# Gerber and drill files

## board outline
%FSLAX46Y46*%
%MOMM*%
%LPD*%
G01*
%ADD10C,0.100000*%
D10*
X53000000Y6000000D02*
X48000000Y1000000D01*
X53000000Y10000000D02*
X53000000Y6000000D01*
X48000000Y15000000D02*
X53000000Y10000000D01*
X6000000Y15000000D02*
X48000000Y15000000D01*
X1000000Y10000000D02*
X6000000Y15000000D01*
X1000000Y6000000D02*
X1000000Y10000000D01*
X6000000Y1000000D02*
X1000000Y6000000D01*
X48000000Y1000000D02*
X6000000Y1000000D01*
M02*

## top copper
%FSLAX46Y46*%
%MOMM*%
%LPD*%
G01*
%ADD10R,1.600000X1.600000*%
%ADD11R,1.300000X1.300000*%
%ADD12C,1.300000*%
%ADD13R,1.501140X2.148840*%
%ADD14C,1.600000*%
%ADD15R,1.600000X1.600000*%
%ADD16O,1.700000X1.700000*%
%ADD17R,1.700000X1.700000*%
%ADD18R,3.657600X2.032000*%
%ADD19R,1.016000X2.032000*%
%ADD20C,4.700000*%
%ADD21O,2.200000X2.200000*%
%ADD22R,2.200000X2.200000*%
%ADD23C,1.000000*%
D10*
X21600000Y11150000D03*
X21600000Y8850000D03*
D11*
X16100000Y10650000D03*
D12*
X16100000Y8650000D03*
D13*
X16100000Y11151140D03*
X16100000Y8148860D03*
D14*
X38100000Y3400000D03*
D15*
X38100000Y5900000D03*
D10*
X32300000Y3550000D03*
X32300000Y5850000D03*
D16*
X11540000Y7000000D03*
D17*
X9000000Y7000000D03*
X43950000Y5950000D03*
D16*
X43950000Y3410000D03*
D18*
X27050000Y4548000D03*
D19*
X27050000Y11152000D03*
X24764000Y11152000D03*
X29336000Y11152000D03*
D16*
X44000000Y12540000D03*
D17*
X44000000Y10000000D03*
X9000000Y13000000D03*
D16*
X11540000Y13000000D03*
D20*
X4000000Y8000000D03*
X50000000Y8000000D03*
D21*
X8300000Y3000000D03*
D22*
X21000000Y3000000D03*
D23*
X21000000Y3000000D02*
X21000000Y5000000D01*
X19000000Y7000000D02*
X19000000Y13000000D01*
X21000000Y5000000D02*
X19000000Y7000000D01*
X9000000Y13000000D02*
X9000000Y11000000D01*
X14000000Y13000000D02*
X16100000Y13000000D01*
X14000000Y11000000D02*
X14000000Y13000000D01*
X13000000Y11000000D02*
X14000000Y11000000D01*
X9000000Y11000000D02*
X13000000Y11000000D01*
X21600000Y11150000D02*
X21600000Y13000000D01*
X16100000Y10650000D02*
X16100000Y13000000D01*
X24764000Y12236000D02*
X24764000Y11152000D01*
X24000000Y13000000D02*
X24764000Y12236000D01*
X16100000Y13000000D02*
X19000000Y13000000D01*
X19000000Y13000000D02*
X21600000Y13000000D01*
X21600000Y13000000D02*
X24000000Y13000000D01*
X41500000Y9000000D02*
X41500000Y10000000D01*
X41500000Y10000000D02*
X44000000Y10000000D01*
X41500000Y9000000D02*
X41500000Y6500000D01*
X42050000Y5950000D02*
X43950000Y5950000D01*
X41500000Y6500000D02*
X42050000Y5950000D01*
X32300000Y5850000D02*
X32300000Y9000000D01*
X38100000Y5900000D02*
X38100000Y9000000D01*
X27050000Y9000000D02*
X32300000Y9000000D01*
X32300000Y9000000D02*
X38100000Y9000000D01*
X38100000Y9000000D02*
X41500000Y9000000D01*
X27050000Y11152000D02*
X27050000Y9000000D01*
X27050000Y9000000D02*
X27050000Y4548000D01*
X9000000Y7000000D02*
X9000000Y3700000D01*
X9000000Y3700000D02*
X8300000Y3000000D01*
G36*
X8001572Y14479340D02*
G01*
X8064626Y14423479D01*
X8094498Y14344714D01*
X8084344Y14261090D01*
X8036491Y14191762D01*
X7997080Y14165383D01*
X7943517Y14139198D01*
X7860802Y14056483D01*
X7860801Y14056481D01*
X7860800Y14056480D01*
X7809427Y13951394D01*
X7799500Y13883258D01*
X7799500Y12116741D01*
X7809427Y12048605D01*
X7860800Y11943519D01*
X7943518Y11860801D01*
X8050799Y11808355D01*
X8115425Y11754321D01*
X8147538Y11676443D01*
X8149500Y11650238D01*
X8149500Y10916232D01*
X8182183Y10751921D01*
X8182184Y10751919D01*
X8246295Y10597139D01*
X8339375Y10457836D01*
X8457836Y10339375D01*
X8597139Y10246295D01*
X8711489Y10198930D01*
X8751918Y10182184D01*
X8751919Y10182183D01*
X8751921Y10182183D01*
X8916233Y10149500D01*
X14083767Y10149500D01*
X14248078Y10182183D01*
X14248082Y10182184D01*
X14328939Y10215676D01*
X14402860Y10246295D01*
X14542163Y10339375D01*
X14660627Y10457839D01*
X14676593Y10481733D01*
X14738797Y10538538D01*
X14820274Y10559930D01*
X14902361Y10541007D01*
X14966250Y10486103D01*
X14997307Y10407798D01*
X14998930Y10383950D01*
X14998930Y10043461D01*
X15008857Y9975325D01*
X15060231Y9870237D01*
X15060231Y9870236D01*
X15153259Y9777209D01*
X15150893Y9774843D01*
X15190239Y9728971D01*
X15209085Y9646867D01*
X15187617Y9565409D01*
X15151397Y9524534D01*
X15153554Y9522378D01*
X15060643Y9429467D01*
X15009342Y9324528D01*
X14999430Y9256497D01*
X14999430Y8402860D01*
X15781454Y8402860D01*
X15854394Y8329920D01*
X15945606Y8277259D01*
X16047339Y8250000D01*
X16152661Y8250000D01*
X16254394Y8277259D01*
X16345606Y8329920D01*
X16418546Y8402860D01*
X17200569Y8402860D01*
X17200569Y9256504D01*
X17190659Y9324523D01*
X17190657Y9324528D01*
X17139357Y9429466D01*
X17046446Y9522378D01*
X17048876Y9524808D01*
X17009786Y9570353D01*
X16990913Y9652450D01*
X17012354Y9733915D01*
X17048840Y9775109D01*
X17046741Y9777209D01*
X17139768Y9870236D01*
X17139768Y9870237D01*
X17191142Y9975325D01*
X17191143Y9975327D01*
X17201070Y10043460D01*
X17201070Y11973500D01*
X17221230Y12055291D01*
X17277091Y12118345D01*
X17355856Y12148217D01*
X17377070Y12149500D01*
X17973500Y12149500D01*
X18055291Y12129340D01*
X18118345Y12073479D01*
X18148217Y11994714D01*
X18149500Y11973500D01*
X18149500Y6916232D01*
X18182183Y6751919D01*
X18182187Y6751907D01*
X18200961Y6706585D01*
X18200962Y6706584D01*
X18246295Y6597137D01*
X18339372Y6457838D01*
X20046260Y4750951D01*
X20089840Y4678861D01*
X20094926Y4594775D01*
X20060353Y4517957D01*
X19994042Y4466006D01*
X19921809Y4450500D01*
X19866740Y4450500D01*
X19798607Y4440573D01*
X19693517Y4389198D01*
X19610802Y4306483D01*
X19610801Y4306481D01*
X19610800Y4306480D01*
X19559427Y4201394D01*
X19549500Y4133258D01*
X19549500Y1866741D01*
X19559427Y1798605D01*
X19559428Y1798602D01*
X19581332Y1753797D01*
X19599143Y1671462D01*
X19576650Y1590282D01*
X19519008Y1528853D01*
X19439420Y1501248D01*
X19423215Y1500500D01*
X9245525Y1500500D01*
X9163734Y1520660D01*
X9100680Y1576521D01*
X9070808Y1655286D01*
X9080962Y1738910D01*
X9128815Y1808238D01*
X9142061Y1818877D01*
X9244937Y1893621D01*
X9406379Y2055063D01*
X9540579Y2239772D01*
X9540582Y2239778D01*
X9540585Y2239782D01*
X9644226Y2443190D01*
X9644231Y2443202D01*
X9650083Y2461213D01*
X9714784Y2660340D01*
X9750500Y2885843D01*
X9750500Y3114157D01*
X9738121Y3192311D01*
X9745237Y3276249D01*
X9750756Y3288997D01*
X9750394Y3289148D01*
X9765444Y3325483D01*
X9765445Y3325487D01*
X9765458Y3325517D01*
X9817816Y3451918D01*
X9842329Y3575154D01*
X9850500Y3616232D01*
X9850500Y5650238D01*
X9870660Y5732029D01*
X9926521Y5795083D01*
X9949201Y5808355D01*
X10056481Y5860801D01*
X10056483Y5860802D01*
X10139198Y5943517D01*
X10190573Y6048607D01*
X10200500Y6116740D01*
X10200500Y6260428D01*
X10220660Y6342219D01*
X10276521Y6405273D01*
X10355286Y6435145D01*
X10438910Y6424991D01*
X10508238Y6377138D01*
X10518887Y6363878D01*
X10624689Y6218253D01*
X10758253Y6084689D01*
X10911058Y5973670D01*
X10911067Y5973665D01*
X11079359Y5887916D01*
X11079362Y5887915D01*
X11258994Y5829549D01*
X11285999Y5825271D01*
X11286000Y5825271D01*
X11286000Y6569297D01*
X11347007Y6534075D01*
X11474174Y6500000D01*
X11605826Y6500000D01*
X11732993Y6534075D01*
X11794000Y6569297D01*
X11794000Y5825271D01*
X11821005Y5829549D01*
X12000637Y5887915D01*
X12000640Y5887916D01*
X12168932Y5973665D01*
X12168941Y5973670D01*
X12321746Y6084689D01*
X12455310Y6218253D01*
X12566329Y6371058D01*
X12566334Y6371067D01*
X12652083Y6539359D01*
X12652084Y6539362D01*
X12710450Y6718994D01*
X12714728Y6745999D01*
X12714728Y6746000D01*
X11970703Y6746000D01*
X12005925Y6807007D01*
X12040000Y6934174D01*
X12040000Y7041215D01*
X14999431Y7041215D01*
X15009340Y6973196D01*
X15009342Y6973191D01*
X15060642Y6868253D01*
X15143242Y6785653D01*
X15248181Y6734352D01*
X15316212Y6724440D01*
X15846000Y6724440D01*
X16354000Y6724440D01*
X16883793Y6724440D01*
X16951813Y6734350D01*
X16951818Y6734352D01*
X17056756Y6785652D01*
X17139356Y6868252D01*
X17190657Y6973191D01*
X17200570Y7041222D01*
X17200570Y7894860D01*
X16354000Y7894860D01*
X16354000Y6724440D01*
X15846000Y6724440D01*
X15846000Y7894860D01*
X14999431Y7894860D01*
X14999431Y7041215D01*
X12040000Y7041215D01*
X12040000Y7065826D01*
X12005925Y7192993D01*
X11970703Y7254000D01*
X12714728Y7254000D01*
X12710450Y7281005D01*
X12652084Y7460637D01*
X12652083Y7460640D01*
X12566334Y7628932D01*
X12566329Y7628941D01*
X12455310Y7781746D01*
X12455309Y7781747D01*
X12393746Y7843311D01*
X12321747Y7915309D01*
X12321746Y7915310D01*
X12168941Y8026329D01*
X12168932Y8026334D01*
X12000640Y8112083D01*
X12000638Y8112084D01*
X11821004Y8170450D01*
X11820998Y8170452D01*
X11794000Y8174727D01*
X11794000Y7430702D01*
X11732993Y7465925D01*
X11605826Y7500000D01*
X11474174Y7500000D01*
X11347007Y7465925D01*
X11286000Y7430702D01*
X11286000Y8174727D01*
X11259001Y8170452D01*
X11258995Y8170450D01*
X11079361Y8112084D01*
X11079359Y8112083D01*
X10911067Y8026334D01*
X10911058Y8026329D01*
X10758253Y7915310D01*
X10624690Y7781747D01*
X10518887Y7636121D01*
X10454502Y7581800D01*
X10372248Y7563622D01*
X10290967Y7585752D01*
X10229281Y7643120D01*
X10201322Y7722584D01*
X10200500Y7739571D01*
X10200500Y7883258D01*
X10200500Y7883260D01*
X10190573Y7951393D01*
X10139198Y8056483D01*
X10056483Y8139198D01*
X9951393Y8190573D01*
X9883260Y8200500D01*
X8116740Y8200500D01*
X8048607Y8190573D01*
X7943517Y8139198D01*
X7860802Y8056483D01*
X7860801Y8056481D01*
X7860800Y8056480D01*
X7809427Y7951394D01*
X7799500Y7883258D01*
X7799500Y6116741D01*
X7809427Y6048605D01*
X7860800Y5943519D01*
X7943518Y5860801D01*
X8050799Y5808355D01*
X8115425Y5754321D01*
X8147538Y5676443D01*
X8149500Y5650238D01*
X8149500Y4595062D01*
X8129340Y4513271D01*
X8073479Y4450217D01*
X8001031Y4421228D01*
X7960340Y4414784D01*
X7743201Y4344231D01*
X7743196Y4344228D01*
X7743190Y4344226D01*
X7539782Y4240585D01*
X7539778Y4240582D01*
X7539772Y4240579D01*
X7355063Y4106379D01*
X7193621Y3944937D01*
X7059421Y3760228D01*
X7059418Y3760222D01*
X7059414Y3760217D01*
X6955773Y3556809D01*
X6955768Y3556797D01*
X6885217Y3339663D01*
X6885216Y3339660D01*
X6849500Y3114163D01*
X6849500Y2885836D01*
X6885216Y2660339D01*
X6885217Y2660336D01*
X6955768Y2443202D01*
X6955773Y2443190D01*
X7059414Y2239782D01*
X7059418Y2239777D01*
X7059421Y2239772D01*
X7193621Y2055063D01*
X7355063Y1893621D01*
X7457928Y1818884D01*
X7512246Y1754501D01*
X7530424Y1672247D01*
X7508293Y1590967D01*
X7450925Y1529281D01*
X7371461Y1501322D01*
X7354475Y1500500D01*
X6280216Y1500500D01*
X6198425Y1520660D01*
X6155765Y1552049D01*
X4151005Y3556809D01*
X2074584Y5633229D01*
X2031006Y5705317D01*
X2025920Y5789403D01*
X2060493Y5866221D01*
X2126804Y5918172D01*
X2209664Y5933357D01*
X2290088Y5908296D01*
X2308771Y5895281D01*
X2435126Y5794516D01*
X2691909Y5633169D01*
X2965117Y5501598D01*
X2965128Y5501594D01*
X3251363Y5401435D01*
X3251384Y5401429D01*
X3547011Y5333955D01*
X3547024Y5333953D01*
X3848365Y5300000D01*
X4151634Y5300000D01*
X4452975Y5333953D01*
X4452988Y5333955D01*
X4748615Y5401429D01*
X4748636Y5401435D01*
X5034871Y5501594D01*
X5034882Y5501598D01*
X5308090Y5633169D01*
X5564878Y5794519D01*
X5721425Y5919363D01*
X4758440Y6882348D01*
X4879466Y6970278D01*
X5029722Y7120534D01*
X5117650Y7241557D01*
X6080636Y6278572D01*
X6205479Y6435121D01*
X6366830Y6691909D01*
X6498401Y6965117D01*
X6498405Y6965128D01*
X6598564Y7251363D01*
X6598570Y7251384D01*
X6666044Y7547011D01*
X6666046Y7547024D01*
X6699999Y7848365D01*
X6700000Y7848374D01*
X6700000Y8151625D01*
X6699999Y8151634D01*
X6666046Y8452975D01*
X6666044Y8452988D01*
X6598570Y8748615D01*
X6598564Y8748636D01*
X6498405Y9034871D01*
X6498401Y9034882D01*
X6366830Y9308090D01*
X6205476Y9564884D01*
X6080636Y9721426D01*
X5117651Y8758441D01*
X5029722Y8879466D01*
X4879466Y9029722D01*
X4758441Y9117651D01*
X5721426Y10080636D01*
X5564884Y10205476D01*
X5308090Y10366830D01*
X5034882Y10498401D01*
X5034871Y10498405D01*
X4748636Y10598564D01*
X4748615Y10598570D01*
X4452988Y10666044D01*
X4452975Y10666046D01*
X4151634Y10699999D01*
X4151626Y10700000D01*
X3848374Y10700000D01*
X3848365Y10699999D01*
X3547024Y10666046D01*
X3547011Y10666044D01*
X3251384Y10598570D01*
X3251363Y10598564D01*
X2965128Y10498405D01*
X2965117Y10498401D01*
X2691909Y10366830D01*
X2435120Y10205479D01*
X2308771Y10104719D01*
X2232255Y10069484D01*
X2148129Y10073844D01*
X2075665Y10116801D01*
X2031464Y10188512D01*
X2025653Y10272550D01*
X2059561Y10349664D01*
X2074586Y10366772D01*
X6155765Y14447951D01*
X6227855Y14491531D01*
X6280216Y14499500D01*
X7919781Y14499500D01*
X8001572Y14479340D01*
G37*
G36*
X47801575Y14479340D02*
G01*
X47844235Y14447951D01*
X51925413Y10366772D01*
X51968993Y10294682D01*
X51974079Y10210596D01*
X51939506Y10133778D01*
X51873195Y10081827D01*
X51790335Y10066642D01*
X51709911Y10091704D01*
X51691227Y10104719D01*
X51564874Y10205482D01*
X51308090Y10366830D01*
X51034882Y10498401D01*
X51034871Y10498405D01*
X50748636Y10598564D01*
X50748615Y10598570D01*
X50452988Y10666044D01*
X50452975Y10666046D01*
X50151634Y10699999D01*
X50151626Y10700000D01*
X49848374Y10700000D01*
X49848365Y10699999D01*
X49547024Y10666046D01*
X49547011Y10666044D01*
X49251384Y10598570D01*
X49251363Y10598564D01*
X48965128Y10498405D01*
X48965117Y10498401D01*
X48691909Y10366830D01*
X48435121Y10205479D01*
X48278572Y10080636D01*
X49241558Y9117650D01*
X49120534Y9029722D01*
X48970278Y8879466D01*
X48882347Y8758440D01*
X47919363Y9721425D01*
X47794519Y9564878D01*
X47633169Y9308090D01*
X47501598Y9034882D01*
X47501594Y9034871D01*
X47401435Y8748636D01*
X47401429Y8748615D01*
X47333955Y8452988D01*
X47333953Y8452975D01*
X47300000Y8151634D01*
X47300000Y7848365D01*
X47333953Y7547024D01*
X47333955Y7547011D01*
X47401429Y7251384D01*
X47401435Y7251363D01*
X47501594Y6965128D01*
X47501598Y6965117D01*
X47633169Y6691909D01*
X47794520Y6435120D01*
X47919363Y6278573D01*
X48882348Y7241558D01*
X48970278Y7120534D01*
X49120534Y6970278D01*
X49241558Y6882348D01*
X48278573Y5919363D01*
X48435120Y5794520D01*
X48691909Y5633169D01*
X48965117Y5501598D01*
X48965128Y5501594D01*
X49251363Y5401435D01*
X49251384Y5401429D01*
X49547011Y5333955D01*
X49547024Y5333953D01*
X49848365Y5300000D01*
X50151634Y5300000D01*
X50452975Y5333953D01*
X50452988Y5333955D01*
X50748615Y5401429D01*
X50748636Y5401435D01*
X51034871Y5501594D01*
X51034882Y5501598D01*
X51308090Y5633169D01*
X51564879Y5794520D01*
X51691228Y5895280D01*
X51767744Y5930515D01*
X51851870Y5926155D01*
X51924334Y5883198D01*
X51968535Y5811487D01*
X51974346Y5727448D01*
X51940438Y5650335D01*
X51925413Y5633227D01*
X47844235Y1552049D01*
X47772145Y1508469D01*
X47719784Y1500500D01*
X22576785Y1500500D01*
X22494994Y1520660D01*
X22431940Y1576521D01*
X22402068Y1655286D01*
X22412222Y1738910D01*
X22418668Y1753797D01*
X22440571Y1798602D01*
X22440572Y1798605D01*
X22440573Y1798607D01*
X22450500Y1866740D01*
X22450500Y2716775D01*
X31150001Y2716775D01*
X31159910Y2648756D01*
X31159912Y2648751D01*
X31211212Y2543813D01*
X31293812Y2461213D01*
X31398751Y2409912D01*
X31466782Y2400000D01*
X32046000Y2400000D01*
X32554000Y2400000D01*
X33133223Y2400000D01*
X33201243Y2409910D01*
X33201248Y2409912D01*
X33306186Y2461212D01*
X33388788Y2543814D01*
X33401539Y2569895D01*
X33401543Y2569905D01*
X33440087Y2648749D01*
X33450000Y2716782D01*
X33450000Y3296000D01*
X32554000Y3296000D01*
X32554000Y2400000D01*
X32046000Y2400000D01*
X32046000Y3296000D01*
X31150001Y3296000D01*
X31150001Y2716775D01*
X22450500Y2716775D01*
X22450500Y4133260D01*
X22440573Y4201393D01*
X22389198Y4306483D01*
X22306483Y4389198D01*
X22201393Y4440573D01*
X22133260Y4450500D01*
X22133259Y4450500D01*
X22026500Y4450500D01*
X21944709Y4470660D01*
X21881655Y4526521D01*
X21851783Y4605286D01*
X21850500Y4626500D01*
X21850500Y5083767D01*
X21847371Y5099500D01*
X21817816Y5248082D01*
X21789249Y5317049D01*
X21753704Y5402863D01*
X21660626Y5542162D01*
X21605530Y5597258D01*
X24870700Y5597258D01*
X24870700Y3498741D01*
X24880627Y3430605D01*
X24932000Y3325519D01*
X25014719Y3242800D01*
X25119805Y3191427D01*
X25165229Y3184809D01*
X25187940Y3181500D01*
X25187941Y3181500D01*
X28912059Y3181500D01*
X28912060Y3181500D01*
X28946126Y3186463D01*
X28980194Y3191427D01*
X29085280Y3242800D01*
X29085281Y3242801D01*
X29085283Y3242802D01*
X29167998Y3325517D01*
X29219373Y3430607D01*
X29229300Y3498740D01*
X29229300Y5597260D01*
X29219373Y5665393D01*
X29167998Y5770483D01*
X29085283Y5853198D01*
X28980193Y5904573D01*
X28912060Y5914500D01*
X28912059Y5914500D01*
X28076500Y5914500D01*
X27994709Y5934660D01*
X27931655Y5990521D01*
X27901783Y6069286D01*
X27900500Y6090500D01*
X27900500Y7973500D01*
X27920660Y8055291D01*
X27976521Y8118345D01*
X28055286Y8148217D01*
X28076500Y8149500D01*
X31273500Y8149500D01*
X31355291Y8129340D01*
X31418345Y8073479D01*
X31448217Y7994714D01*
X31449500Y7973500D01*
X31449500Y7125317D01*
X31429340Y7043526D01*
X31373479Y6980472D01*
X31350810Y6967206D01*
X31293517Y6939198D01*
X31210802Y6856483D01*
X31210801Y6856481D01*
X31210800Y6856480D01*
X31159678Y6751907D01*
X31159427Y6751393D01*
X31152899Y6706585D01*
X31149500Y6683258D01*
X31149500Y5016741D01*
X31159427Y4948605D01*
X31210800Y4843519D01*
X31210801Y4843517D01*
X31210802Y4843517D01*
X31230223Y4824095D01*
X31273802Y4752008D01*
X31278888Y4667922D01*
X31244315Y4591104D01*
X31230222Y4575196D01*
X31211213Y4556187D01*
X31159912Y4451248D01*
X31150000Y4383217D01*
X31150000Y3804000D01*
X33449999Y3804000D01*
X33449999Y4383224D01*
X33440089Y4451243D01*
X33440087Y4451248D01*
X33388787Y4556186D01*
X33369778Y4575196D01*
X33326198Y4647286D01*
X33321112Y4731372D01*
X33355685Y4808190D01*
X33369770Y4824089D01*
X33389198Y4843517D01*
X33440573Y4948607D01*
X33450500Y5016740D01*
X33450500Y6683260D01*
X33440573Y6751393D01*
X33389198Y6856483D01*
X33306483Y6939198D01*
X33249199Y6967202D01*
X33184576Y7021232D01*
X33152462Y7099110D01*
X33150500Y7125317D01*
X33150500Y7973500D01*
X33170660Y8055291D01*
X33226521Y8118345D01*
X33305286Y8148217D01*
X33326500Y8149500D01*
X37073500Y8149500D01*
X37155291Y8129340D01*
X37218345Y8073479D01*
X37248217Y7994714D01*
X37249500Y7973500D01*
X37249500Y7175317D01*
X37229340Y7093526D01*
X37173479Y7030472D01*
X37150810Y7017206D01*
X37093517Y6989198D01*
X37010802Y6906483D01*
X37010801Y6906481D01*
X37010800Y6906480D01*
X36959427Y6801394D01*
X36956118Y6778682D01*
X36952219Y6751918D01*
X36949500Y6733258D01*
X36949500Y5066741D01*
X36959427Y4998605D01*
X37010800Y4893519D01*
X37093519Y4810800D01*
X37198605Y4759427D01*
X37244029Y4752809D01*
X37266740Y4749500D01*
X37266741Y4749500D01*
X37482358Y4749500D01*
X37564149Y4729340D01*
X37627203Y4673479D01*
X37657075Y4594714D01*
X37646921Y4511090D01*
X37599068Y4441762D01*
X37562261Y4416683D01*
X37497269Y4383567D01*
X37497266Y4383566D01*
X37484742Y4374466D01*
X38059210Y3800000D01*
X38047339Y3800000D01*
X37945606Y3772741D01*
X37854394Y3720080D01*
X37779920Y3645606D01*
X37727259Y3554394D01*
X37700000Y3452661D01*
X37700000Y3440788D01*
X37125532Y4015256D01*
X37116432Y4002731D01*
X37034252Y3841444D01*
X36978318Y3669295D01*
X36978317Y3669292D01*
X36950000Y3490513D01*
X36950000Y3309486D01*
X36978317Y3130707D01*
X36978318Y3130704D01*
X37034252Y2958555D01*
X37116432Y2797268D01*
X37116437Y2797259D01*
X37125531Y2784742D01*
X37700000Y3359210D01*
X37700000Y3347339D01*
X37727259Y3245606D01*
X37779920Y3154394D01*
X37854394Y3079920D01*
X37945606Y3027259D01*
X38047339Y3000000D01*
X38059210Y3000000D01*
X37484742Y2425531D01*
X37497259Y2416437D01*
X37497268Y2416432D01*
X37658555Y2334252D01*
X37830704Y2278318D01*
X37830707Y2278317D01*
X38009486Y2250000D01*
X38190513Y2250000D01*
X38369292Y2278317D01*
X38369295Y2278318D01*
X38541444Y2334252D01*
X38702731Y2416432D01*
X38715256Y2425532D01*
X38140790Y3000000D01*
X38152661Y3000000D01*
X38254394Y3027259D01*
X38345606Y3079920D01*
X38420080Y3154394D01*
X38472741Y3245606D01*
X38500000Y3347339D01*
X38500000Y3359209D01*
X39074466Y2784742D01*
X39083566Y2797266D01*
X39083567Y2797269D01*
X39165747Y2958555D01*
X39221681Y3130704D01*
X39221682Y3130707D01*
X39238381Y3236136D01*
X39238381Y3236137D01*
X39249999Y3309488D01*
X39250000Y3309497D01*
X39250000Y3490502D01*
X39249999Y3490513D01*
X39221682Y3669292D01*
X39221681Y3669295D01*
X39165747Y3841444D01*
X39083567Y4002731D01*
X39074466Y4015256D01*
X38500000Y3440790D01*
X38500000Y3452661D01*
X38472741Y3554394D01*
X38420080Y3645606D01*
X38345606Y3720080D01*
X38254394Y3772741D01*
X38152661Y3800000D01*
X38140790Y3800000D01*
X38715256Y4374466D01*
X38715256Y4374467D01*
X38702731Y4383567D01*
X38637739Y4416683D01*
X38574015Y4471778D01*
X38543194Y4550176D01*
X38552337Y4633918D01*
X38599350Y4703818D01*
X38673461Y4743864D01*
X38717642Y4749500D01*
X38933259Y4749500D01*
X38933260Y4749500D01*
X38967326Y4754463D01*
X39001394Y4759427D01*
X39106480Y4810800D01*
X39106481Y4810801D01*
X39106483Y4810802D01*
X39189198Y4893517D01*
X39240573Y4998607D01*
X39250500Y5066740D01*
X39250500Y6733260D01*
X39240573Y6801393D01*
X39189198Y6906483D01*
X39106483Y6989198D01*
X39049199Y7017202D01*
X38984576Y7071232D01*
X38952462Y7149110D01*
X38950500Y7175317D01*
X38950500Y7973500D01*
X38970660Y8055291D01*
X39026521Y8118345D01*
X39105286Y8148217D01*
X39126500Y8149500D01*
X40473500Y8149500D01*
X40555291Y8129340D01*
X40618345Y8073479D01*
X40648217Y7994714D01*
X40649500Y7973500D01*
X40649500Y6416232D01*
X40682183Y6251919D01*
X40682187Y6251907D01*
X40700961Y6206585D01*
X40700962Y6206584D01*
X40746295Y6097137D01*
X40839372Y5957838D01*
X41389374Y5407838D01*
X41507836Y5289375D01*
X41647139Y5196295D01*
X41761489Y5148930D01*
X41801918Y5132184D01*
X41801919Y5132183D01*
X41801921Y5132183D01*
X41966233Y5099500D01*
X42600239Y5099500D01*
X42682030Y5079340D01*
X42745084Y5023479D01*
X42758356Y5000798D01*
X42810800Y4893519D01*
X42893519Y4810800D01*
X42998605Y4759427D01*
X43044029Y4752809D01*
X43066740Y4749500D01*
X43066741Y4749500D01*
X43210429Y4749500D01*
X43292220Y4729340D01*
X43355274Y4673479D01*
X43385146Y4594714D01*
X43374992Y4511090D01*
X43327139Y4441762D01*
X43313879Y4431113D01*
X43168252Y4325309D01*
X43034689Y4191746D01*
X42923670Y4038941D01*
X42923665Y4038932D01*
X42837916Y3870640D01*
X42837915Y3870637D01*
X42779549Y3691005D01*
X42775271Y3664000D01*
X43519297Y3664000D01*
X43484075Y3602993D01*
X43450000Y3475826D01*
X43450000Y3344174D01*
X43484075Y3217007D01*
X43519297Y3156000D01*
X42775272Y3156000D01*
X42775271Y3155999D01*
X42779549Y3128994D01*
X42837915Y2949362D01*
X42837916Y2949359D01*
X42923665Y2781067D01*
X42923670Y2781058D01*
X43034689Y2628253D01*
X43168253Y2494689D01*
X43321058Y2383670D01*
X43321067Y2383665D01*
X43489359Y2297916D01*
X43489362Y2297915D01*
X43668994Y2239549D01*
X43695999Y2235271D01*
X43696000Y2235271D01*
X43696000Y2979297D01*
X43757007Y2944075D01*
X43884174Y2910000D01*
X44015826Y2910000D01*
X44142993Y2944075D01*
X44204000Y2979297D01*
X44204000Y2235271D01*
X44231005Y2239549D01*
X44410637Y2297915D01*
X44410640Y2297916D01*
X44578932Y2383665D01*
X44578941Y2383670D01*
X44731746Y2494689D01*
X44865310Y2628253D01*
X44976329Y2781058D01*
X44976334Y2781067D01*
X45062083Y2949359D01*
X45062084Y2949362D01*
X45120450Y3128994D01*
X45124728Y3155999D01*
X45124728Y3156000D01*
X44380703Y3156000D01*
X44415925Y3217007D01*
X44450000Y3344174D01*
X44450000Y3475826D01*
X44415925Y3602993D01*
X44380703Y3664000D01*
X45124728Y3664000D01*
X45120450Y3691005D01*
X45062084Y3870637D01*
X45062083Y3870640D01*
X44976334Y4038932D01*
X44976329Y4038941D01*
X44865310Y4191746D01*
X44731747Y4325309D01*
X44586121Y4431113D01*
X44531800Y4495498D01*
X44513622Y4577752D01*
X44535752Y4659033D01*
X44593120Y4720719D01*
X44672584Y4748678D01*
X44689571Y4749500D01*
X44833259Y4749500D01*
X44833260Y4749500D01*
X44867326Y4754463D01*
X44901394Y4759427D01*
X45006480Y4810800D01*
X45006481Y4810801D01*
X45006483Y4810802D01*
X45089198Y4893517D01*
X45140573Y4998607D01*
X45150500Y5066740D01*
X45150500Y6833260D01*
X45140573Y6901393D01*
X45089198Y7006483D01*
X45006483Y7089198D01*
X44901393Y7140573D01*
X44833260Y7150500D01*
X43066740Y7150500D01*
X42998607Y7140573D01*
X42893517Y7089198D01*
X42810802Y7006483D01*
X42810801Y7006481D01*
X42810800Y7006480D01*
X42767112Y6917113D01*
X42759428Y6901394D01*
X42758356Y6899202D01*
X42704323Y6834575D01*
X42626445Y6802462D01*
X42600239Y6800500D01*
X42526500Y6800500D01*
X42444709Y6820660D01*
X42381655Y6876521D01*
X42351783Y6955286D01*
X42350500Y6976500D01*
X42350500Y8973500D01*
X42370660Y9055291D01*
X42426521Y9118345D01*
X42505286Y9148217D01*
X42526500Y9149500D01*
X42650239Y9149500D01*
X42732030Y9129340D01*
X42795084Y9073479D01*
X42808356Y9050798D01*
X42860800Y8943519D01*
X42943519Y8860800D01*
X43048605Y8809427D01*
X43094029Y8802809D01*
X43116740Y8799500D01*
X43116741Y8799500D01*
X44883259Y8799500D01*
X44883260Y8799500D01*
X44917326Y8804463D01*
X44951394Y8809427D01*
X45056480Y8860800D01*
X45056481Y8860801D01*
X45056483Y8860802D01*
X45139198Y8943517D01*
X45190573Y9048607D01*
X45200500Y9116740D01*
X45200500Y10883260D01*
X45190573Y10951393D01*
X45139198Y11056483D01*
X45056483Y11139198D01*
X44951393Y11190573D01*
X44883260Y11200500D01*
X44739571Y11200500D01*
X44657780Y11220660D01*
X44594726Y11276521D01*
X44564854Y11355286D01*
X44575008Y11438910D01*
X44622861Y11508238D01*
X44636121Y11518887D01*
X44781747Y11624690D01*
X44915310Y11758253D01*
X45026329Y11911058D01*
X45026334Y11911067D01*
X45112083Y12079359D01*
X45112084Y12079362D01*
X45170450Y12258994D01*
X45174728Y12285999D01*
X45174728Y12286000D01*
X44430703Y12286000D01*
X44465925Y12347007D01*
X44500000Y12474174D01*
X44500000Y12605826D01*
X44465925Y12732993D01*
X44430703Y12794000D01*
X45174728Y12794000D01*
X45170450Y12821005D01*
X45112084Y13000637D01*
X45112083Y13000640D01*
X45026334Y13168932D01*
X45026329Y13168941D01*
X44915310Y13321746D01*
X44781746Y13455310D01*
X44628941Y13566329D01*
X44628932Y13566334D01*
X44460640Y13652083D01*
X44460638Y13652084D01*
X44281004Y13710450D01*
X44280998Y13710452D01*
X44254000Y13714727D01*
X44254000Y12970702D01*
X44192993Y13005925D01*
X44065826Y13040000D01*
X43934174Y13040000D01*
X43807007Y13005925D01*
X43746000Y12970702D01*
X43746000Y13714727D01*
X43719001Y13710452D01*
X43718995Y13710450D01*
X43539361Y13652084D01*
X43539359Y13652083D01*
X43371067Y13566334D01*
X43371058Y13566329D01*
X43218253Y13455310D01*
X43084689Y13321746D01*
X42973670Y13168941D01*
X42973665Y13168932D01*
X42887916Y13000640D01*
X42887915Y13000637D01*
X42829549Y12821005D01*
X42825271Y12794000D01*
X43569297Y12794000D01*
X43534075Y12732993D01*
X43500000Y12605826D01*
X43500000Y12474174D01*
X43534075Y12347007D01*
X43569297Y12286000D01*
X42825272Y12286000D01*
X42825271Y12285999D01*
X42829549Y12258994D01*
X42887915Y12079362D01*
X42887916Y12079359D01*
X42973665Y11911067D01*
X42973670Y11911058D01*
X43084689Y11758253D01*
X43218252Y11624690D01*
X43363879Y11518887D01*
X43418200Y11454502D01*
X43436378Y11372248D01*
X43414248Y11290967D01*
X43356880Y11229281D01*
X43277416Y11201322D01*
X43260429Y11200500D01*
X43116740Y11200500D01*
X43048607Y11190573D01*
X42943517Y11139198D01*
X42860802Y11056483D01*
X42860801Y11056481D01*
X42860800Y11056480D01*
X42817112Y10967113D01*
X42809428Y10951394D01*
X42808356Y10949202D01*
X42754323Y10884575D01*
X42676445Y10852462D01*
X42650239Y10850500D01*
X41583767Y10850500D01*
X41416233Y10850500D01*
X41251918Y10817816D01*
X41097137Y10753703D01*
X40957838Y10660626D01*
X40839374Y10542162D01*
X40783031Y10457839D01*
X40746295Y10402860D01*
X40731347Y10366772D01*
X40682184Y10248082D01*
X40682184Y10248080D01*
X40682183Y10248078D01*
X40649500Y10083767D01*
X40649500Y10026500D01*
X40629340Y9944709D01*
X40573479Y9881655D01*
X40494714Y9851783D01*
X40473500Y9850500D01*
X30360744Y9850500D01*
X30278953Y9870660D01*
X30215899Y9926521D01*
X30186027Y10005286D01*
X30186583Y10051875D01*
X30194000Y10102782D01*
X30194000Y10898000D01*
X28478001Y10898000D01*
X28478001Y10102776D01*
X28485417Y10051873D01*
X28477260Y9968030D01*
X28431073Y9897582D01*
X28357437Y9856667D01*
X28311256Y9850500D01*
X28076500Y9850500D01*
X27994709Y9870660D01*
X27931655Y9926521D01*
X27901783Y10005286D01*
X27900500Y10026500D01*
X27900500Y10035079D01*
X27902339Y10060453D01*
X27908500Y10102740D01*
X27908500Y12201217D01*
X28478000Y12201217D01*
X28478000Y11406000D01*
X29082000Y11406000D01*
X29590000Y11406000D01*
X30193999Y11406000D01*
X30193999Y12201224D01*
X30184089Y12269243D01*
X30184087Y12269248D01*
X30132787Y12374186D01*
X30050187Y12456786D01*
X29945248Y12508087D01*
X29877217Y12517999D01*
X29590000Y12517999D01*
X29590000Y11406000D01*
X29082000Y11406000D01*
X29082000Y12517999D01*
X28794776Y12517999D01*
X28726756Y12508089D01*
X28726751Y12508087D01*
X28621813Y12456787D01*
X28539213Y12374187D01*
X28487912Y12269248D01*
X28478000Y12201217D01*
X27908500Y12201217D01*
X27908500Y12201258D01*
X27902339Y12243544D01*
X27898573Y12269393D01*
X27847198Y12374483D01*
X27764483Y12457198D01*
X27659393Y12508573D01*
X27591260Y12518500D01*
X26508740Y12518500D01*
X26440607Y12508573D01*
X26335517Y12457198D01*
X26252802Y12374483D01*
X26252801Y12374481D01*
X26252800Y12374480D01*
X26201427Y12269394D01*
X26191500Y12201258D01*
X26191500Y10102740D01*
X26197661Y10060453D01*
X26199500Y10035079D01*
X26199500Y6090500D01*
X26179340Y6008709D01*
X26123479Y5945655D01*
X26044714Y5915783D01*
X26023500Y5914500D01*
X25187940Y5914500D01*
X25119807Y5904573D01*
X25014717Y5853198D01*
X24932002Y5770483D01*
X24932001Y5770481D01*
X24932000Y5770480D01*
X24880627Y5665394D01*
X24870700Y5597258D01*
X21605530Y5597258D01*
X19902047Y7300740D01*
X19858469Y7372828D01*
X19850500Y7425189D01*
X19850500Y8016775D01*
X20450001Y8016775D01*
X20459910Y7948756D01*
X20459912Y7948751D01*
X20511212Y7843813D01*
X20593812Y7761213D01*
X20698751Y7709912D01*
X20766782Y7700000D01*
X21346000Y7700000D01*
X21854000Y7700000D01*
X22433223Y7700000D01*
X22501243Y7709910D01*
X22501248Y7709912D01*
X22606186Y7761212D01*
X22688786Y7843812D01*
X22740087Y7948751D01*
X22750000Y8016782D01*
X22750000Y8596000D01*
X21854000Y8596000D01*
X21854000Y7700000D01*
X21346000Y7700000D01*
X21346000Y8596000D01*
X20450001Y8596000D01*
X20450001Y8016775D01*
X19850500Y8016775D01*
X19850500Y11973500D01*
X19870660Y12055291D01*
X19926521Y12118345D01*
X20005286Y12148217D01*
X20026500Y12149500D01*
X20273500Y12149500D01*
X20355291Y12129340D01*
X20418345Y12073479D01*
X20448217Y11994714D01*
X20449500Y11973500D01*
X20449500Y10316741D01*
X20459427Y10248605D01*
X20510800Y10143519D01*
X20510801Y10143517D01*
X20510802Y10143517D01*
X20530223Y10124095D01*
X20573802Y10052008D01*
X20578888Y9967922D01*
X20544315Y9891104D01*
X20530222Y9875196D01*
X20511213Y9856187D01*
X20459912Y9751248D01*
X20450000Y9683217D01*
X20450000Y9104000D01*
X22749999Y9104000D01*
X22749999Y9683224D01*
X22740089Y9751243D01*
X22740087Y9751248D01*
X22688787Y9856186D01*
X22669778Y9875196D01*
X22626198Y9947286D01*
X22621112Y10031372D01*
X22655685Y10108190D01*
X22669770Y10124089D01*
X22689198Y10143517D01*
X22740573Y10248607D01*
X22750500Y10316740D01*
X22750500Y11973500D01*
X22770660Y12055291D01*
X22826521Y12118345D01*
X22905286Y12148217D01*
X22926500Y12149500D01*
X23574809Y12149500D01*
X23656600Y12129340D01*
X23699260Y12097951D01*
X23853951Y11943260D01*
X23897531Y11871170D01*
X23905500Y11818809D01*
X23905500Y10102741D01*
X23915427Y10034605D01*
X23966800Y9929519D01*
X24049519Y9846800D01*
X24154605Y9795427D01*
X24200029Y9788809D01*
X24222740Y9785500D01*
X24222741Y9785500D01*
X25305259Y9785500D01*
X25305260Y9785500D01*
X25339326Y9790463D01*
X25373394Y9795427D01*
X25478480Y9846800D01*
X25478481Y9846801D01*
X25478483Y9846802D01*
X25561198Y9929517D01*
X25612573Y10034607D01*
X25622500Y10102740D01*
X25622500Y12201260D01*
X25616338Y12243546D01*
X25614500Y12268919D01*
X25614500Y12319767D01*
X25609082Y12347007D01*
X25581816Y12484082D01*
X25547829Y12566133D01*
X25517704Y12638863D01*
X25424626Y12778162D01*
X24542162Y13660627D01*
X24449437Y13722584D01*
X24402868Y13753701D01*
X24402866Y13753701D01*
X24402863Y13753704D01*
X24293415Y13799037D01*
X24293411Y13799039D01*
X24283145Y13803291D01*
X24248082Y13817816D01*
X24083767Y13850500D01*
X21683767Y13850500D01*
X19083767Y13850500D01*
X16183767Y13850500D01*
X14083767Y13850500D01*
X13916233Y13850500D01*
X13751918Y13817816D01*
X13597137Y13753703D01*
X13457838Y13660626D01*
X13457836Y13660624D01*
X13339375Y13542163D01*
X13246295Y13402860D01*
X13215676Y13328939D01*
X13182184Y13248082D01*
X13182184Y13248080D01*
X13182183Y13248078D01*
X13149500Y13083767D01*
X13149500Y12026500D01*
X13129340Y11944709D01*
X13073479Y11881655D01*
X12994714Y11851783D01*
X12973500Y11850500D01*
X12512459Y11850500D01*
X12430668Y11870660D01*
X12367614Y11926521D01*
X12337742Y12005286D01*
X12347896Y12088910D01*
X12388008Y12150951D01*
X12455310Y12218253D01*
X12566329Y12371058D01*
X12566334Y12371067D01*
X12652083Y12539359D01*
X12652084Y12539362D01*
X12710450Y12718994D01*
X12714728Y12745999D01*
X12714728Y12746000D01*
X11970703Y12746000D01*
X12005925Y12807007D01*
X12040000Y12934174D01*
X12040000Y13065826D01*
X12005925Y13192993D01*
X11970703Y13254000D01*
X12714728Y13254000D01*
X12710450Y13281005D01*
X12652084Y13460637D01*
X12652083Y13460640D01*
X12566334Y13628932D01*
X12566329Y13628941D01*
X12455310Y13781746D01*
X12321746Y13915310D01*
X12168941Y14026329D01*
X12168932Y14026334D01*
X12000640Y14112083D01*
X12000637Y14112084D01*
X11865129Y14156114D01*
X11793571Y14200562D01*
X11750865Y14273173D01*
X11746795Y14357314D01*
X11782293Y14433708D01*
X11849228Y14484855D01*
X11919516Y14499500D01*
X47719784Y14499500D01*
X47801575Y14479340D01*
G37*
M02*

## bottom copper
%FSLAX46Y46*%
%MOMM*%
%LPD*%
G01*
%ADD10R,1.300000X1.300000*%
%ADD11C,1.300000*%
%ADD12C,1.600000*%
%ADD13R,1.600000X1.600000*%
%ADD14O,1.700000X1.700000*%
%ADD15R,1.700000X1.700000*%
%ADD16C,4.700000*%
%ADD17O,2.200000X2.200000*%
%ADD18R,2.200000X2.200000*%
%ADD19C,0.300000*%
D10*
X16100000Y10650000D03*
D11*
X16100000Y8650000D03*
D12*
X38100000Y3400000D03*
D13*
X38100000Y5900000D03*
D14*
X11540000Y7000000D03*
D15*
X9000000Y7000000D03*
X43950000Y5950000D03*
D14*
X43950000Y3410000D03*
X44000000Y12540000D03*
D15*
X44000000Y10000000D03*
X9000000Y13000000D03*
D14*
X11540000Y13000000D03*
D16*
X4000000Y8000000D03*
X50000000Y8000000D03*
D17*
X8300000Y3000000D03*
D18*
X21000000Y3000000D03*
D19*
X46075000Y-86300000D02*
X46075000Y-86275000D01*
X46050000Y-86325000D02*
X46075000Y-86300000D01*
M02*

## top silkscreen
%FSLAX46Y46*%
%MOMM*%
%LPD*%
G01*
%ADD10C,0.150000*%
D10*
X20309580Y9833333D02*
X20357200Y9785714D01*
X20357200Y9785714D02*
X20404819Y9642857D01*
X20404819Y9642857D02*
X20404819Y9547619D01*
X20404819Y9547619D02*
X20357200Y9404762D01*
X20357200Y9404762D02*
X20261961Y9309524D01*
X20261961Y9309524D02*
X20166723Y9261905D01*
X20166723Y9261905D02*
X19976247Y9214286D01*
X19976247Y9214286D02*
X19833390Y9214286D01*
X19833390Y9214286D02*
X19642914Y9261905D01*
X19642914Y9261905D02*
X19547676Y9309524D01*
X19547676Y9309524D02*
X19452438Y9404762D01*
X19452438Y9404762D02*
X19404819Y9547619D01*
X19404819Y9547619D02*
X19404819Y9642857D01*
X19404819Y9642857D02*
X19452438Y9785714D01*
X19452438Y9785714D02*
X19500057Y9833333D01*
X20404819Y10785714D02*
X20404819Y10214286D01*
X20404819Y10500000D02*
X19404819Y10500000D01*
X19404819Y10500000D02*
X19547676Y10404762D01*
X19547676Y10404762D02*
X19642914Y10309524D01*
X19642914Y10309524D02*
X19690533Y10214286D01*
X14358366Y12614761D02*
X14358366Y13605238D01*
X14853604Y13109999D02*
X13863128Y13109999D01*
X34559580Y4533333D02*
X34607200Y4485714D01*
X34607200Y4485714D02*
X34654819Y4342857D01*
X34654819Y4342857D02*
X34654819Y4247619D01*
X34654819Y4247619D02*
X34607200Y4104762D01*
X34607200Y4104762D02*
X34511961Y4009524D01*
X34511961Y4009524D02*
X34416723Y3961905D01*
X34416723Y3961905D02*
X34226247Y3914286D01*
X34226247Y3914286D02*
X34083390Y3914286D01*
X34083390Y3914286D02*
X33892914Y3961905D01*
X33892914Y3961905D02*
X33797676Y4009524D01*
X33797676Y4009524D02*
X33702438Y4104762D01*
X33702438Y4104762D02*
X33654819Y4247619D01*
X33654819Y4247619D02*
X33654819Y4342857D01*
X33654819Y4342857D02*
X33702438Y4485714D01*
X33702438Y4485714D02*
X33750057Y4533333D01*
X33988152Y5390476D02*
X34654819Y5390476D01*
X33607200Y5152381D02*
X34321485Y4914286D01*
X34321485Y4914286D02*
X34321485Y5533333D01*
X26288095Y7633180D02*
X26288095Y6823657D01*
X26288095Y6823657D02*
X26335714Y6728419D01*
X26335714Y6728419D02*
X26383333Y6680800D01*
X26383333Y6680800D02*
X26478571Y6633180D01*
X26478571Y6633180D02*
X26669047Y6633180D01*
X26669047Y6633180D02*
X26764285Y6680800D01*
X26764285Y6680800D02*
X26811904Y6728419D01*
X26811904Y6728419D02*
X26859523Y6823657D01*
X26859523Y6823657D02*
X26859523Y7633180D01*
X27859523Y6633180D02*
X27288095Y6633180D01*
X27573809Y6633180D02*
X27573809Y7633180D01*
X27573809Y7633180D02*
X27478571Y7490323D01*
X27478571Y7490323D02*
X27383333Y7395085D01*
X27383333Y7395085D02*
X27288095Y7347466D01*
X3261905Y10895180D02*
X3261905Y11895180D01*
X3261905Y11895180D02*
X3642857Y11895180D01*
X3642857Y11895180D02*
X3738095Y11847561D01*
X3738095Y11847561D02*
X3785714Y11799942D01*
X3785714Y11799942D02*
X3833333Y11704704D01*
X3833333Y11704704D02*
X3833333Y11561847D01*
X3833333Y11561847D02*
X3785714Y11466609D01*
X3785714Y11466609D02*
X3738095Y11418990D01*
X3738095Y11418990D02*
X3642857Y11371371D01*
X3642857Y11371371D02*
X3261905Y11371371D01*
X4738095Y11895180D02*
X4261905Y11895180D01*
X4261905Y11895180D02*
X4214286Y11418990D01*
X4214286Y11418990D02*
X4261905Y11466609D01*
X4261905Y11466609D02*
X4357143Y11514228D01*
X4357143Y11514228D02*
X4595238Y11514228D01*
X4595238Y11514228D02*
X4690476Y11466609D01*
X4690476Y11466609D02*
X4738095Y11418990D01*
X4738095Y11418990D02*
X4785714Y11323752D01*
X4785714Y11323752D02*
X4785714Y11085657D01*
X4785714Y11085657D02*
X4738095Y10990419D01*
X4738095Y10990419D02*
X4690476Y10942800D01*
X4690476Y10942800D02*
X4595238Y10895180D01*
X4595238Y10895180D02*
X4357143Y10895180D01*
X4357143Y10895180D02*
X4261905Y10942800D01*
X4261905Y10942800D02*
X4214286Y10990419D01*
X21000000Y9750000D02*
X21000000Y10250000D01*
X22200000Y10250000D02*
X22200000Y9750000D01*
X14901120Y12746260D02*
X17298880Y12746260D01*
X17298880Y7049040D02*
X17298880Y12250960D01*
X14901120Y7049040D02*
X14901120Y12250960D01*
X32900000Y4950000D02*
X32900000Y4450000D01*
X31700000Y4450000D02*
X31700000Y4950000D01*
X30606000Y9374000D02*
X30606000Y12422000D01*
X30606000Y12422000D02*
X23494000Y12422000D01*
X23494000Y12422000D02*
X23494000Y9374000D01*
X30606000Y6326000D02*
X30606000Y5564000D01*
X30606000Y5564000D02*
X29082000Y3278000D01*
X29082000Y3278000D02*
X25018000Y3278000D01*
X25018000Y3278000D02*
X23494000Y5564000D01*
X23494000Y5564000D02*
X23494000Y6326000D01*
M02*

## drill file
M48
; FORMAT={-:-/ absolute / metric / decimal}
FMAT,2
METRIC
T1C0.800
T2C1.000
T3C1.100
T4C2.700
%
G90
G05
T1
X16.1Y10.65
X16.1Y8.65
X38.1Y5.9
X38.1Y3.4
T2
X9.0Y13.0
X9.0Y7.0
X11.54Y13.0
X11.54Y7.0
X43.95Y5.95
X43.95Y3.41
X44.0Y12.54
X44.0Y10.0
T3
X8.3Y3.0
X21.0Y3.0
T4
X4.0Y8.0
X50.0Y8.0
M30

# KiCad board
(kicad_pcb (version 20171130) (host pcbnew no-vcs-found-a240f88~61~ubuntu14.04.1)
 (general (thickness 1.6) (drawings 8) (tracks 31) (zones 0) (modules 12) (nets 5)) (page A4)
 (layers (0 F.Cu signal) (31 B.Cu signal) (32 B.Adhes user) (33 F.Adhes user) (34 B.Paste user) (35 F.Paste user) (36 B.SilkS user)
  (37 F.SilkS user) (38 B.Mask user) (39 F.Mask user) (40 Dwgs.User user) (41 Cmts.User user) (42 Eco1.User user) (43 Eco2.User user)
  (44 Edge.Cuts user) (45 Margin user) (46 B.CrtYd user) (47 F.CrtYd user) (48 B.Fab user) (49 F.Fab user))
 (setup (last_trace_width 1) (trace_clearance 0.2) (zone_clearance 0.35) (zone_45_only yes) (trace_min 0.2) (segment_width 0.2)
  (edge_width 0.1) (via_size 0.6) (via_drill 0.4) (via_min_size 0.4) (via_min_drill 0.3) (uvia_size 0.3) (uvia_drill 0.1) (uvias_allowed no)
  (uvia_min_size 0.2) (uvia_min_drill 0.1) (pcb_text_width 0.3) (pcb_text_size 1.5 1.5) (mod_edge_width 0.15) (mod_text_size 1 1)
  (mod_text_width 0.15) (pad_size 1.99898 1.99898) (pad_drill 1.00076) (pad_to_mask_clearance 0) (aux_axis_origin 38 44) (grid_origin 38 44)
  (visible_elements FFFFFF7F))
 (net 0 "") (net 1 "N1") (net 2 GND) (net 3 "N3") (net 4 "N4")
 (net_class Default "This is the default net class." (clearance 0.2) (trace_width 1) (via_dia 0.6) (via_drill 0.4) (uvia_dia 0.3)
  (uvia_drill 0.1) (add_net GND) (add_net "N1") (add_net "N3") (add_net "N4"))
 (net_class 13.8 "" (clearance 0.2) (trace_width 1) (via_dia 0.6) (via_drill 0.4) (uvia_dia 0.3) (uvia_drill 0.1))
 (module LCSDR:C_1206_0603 (layer F.Cu) (at 21.6 -10 270)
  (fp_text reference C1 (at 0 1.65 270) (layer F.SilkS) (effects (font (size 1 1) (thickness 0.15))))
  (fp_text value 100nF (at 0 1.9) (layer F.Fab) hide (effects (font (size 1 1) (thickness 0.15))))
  (fp_line (start 0.25 0.6) (end -0.25 0.6) (layer F.SilkS) (width 0.15))
  (fp_line (start -0.25 -0.6) (end 0.25 -0.6) (layer F.SilkS) (width 0.15))
  (pad 1 smd rect (at -1.15 0 270) (size 1.6 1.6) (layers F.Cu F.Paste F.Mask) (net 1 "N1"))
  (pad 2 smd rect (at 1.15 0 270) (size 1.6 1.6) (layers F.Cu F.Paste F.Mask) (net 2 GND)))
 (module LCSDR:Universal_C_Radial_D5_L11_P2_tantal (layer B.Cu) (at 16.1 -9.65 270)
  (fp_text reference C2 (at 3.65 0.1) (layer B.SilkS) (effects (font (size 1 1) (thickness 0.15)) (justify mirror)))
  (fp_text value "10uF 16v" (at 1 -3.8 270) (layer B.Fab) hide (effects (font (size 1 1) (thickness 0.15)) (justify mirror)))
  (fp_line (start -3.09626 1.19888) (end -3.09626 -1.19888) (layer F.SilkS) (width 0.15))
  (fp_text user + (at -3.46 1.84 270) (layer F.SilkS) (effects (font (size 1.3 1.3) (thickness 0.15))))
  (fp_line (start 2.60096 -1.19888) (end -2.60096 -1.19888) (layer F.SilkS) (width 0.15))
  (fp_line (start 2.60096 1.19888) (end -2.60096 1.19888) (layer F.SilkS) (width 0.15))
  (pad 1 thru_hole rect (at -1 0 270) (size 1.3 1.3) (drill 0.8) (layers *.Cu *.Mask B.SilkS) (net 1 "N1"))
  (pad 2 thru_hole circle (at 1 0 270) (size 1.3 1.3) (drill 0.8) (layers *.Cu *.Mask B.SilkS) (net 2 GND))
  (pad 1 smd rect (at -1.50114 0 270) (size 2.14884 1.50114) (layers F.Cu F.Paste F.Mask) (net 1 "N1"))
  (pad 2 smd rect (at 1.50114 0 270) (size 2.14884 1.50114) (layers F.Cu F.Paste F.Mask) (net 2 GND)))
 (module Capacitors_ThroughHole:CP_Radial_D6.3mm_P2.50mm (layer B.Cu) (at 38.1 -5.9 270)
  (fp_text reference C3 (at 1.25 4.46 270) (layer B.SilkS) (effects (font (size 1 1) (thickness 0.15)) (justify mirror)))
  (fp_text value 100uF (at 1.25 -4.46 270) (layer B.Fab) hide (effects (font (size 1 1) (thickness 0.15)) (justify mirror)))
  (pad 2 thru_hole circle (at 2.5 0 270) (size 1.6 1.6) (drill 0.8) (layers *.Cu *.Mask) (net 2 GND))
  (pad 1 thru_hole rect (at 0 0 270) (size 1.6 1.6) (drill 0.8) (layers *.Cu *.Mask) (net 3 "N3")))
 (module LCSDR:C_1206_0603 (layer F.Cu) (at 32.3 -4.7 270)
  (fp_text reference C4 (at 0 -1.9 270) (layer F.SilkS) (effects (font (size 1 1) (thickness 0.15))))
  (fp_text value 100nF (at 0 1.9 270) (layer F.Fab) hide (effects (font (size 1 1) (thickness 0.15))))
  (fp_line (start -0.25 -0.6) (end 0.25 -0.6) (layer F.SilkS) (width 0.15))
  (fp_line (start 0.25 0.6) (end -0.25 0.6) (layer F.SilkS) (width 0.15))
  (pad 2 smd rect (at 1.15 0 270) (size 1.6 1.6) (layers F.Cu F.Paste F.Mask) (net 2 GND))
  (pad 1 smd rect (at -1.15 0 270) (size 1.6 1.6) (layers F.Cu F.Paste F.Mask) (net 3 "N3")))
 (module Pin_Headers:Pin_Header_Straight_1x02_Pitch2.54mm (layer B.Cu) (at 9 -7 270)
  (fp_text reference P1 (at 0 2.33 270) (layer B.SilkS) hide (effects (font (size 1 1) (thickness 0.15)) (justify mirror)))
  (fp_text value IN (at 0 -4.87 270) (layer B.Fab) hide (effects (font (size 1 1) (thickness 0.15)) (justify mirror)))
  (pad 2 thru_hole oval (at 0 -2.54 270) (size 1.7 1.7) (drill 1) (layers *.Cu *.Mask) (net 2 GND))
  (pad 1 thru_hole rect (at 0 0 270) (size 1.7 1.7) (drill 1) (layers *.Cu *.Mask) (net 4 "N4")))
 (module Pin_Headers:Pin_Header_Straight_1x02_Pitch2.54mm (layer B.Cu) (at 43.95 -5.95 180)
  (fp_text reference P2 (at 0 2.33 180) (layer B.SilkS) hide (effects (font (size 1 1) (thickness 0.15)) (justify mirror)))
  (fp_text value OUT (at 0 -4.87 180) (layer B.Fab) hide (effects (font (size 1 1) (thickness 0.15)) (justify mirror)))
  (pad 1 thru_hole rect (at 0 0 180) (size 1.7 1.7) (drill 1) (layers *.Cu *.Mask) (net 3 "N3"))
  (pad 2 thru_hole oval (at 0 -2.54 180) (size 1.7 1.7) (drill 1) (layers *.Cu *.Mask) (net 2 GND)))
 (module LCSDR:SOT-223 (layer F.Cu) (at 27.05 -7.85 180)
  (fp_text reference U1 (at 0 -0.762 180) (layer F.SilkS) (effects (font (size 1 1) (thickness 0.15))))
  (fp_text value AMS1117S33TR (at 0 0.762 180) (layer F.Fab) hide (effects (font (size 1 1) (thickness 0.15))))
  (fp_line (start -3.556 1.524) (end -3.556 4.572) (layer F.SilkS) (width 0.15))
  (fp_line (start -3.556 4.572) (end 3.556 4.572) (layer F.SilkS) (width 0.15))
  (fp_line (start 3.556 4.572) (end 3.556 1.524) (layer F.SilkS) (width 0.15))
  (fp_line (start -3.556 -1.524) (end -3.556 -2.286) (layer F.SilkS) (width 0.15))
  (fp_line (start -3.556 -2.286) (end -2.032 -4.572) (layer F.SilkS) (width 0.15))
  (fp_line (start -2.032 -4.572) (end 2.032 -4.572) (layer F.SilkS) (width 0.15))
  (fp_line (start 2.032 -4.572) (end 3.556 -2.286) (layer F.SilkS) (width 0.15))
  (fp_line (start 3.556 -2.286) (end 3.556 -1.524) (layer F.SilkS) (width 0.15))
  (pad 4 smd rect (at 0 -3.302 180) (size 3.6576 2.032) (layers F.Cu F.Paste F.Mask) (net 3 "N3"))
  (pad 2 smd rect (at 0 3.302 180) (size 1.016 2.032) (layers F.Cu F.Paste F.Mask) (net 3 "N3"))
  (pad 3 smd rect (at 2.286 3.302 180) (size 1.016 2.032) (layers F.Cu F.Paste F.Mask) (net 1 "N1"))
  (pad 1 smd rect (at -2.286 3.302 180) (size 1.016 2.032) (layers F.Cu F.Paste F.Mask) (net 2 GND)))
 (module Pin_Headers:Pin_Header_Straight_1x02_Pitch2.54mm (layer B.Cu) (at 44 -10)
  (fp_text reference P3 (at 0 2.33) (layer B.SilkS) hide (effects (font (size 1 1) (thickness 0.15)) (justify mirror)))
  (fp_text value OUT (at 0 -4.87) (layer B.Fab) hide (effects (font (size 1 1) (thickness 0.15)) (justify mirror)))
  (pad 2 thru_hole oval (at 0 -2.54) (size 1.7 1.7) (drill 1) (layers *.Cu *.Mask) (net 2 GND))
  (pad 1 thru_hole rect (at 0 0) (size 1.7 1.7) (drill 1) (layers *.Cu *.Mask) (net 3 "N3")))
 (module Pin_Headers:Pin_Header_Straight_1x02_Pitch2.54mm (layer B.Cu) (at 9 -13 270)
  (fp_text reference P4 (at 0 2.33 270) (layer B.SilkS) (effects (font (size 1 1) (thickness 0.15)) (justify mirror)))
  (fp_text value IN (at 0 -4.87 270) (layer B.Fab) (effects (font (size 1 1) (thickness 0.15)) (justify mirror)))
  (pad 1 thru_hole rect (at 0 0 270) (size 1.7 1.7) (drill 1) (layers *.Cu *.Mask) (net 1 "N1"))
  (pad 2 thru_hole oval (at 0 -2.54 270) (size 1.7 1.7) (drill 1) (layers *.Cu *.Mask) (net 2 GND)))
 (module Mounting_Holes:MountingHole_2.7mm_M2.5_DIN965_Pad (layer F.Cu) (at 4 -8)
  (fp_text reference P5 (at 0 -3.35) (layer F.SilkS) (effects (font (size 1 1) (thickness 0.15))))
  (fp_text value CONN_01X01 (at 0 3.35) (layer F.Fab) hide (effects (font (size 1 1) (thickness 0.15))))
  (pad 1 thru_hole circle (at 0 0) (size 4.7 4.7) (drill 2.7) (layers *.Cu *.Mask) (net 2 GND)))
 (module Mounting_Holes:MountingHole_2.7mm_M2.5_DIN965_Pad (layer F.Cu) (at 50 -8)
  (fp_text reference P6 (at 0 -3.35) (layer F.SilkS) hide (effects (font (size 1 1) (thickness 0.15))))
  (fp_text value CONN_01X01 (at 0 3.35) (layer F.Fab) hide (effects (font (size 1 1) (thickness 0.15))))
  (pad 1 thru_hole circle (at 0 0) (size 4.7 4.7) (drill 2.7) (layers *.Cu *.Mask) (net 2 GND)))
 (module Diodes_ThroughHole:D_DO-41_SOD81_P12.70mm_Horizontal (layer B.Cu) (at 21 -3 180)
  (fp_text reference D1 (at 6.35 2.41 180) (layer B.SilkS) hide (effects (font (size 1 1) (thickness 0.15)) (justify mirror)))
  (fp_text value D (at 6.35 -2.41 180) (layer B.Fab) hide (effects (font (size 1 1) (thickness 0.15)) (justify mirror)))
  (pad 2 thru_hole oval (at 12.7 0 180) (size 2.2 2.2) (drill 1.1) (layers *.Cu *.Mask) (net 4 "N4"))
  (pad 1 thru_hole rect (at 0 0 180) (size 2.2 2.2) (drill 1.1) (layers *.Cu *.Mask) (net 1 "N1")))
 (gr_line (start 53 -6) (end 48 -1) (angle 90) (layer Edge.Cuts) (width 0.1))
 (gr_line (start 53 -10) (end 53 -6) (angle 90) (layer Edge.Cuts) (width 0.1))
 (gr_line (start 48 -15) (end 53 -10) (angle 90) (layer Edge.Cuts) (width 0.1))
 (gr_line (start 6 -15) (end 48 -15) (angle 90) (layer Edge.Cuts) (width 0.1))
 (gr_line (start 1 -10) (end 6 -15) (angle 90) (layer Edge.Cuts) (width 0.1))
 (gr_line (start 1 -6) (end 1 -10) (angle 90) (layer Edge.Cuts) (width 0.1))
 (gr_line (start 6 -1) (end 1 -6) (angle 90) (layer Edge.Cuts) (width 0.1))
 (gr_line (start 48 -1) (end 6 -1) (angle 90) (layer Edge.Cuts) (width 0.1))
 (segment (start 46.075 86.3) (end 46.075 86.275) (width 0.3) (layer B.Cu) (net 2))
 (segment (start 46.05 86.325) (end 46.075 86.3) (width 0.3) (layer B.Cu) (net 2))
 (segment (start 21 -3) (end 21 -5) (width 1) (layer F.Cu) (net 1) (status 400000))
 (segment (start 19 -7) (end 19 -13) (width 1) (layer F.Cu) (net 1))
 (segment (start 21 -5) (end 19 -7) (width 1) (layer F.Cu) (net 1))
 (segment (start 9 -13) (end 9 -11) (width 1) (layer F.Cu) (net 1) (status 400000))
 (segment (start 14 -13) (end 16.1 -13) (width 1) (layer F.Cu) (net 1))
 (segment (start 14 -11) (end 14 -13) (width 1) (layer F.Cu) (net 1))
 (segment (start 13 -11) (end 14 -11) (width 1) (layer F.Cu) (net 1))
 (segment (start 9 -11) (end 13 -11) (width 1) (layer F.Cu) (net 1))
 (segment (start 21.6 -11.15) (end 21.6 -13) (width 1) (layer F.Cu) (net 1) (status 400000))
 (segment (start 16.1 -10.65) (end 16.1 -13) (width 1) (layer F.Cu) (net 1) (status 400000))
 (segment (start 24.764 -12.236) (end 24.764 -11.152) (width 1) (layer F.Cu) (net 1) (status 800000))
 (segment (start 24 -13) (end 24.764 -12.236) (width 1) (layer F.Cu) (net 1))
 (segment (start 16.1 -13) (end 19 -13) (width 1) (layer F.Cu) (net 1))
 (segment (start 19 -13) (end 21.6 -13) (width 1) (layer F.Cu) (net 1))
 (segment (start 21.6 -13) (end 24 -13) (width 1) (layer F.Cu) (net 1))
 (segment (start 41.5 -9) (end 41.5 -10) (width 1) (layer F.Cu) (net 3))
 (segment (start 41.5 -10) (end 44 -10) (width 1) (layer F.Cu) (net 3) (status 800000))
 (segment (start 41.5 -9) (end 41.5 -6.5) (width 1) (layer F.Cu) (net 3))
 (segment (start 42.05 -5.95) (end 43.95 -5.95) (width 1) (layer F.Cu) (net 3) (status 800000))
 (segment (start 41.5 -6.5) (end 42.05 -5.95) (width 1) (layer F.Cu) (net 3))
 (segment (start 32.3 -5.85) (end 32.3 -9) (width 1) (layer F.Cu) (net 3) (status 400000))
 (segment (start 38.1 -5.9) (end 38.1 -9) (width 1) (layer F.Cu) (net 3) (status 400000))
 (segment (start 27.05 -9) (end 32.3 -9) (width 1) (layer F.Cu) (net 3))
 (segment (start 32.3 -9) (end 38.1 -9) (width 1) (layer F.Cu) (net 3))
 (segment (start 38.1 -9) (end 41.5 -9) (width 1) (layer F.Cu) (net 3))
 (segment (start 27.05 -11.152) (end 27.05 -9) (width 1) (layer F.Cu) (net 3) (status 400000))
 (segment (start 27.05 -9) (end 27.05 -4.548) (width 1) (layer F.Cu) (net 3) (status 800000))
 (segment (start 9 -7) (end 9 -3.7) (width 1) (layer F.Cu) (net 4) (status C00000))
 (segment (start 9 -3.7) (end 8.3 -3) (width 1) (layer F.Cu) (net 4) (status C00000))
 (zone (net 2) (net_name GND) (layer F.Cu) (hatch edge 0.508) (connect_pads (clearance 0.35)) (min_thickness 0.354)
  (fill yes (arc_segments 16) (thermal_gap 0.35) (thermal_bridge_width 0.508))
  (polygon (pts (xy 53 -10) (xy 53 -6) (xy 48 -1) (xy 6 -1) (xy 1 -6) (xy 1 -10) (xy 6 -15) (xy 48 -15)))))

